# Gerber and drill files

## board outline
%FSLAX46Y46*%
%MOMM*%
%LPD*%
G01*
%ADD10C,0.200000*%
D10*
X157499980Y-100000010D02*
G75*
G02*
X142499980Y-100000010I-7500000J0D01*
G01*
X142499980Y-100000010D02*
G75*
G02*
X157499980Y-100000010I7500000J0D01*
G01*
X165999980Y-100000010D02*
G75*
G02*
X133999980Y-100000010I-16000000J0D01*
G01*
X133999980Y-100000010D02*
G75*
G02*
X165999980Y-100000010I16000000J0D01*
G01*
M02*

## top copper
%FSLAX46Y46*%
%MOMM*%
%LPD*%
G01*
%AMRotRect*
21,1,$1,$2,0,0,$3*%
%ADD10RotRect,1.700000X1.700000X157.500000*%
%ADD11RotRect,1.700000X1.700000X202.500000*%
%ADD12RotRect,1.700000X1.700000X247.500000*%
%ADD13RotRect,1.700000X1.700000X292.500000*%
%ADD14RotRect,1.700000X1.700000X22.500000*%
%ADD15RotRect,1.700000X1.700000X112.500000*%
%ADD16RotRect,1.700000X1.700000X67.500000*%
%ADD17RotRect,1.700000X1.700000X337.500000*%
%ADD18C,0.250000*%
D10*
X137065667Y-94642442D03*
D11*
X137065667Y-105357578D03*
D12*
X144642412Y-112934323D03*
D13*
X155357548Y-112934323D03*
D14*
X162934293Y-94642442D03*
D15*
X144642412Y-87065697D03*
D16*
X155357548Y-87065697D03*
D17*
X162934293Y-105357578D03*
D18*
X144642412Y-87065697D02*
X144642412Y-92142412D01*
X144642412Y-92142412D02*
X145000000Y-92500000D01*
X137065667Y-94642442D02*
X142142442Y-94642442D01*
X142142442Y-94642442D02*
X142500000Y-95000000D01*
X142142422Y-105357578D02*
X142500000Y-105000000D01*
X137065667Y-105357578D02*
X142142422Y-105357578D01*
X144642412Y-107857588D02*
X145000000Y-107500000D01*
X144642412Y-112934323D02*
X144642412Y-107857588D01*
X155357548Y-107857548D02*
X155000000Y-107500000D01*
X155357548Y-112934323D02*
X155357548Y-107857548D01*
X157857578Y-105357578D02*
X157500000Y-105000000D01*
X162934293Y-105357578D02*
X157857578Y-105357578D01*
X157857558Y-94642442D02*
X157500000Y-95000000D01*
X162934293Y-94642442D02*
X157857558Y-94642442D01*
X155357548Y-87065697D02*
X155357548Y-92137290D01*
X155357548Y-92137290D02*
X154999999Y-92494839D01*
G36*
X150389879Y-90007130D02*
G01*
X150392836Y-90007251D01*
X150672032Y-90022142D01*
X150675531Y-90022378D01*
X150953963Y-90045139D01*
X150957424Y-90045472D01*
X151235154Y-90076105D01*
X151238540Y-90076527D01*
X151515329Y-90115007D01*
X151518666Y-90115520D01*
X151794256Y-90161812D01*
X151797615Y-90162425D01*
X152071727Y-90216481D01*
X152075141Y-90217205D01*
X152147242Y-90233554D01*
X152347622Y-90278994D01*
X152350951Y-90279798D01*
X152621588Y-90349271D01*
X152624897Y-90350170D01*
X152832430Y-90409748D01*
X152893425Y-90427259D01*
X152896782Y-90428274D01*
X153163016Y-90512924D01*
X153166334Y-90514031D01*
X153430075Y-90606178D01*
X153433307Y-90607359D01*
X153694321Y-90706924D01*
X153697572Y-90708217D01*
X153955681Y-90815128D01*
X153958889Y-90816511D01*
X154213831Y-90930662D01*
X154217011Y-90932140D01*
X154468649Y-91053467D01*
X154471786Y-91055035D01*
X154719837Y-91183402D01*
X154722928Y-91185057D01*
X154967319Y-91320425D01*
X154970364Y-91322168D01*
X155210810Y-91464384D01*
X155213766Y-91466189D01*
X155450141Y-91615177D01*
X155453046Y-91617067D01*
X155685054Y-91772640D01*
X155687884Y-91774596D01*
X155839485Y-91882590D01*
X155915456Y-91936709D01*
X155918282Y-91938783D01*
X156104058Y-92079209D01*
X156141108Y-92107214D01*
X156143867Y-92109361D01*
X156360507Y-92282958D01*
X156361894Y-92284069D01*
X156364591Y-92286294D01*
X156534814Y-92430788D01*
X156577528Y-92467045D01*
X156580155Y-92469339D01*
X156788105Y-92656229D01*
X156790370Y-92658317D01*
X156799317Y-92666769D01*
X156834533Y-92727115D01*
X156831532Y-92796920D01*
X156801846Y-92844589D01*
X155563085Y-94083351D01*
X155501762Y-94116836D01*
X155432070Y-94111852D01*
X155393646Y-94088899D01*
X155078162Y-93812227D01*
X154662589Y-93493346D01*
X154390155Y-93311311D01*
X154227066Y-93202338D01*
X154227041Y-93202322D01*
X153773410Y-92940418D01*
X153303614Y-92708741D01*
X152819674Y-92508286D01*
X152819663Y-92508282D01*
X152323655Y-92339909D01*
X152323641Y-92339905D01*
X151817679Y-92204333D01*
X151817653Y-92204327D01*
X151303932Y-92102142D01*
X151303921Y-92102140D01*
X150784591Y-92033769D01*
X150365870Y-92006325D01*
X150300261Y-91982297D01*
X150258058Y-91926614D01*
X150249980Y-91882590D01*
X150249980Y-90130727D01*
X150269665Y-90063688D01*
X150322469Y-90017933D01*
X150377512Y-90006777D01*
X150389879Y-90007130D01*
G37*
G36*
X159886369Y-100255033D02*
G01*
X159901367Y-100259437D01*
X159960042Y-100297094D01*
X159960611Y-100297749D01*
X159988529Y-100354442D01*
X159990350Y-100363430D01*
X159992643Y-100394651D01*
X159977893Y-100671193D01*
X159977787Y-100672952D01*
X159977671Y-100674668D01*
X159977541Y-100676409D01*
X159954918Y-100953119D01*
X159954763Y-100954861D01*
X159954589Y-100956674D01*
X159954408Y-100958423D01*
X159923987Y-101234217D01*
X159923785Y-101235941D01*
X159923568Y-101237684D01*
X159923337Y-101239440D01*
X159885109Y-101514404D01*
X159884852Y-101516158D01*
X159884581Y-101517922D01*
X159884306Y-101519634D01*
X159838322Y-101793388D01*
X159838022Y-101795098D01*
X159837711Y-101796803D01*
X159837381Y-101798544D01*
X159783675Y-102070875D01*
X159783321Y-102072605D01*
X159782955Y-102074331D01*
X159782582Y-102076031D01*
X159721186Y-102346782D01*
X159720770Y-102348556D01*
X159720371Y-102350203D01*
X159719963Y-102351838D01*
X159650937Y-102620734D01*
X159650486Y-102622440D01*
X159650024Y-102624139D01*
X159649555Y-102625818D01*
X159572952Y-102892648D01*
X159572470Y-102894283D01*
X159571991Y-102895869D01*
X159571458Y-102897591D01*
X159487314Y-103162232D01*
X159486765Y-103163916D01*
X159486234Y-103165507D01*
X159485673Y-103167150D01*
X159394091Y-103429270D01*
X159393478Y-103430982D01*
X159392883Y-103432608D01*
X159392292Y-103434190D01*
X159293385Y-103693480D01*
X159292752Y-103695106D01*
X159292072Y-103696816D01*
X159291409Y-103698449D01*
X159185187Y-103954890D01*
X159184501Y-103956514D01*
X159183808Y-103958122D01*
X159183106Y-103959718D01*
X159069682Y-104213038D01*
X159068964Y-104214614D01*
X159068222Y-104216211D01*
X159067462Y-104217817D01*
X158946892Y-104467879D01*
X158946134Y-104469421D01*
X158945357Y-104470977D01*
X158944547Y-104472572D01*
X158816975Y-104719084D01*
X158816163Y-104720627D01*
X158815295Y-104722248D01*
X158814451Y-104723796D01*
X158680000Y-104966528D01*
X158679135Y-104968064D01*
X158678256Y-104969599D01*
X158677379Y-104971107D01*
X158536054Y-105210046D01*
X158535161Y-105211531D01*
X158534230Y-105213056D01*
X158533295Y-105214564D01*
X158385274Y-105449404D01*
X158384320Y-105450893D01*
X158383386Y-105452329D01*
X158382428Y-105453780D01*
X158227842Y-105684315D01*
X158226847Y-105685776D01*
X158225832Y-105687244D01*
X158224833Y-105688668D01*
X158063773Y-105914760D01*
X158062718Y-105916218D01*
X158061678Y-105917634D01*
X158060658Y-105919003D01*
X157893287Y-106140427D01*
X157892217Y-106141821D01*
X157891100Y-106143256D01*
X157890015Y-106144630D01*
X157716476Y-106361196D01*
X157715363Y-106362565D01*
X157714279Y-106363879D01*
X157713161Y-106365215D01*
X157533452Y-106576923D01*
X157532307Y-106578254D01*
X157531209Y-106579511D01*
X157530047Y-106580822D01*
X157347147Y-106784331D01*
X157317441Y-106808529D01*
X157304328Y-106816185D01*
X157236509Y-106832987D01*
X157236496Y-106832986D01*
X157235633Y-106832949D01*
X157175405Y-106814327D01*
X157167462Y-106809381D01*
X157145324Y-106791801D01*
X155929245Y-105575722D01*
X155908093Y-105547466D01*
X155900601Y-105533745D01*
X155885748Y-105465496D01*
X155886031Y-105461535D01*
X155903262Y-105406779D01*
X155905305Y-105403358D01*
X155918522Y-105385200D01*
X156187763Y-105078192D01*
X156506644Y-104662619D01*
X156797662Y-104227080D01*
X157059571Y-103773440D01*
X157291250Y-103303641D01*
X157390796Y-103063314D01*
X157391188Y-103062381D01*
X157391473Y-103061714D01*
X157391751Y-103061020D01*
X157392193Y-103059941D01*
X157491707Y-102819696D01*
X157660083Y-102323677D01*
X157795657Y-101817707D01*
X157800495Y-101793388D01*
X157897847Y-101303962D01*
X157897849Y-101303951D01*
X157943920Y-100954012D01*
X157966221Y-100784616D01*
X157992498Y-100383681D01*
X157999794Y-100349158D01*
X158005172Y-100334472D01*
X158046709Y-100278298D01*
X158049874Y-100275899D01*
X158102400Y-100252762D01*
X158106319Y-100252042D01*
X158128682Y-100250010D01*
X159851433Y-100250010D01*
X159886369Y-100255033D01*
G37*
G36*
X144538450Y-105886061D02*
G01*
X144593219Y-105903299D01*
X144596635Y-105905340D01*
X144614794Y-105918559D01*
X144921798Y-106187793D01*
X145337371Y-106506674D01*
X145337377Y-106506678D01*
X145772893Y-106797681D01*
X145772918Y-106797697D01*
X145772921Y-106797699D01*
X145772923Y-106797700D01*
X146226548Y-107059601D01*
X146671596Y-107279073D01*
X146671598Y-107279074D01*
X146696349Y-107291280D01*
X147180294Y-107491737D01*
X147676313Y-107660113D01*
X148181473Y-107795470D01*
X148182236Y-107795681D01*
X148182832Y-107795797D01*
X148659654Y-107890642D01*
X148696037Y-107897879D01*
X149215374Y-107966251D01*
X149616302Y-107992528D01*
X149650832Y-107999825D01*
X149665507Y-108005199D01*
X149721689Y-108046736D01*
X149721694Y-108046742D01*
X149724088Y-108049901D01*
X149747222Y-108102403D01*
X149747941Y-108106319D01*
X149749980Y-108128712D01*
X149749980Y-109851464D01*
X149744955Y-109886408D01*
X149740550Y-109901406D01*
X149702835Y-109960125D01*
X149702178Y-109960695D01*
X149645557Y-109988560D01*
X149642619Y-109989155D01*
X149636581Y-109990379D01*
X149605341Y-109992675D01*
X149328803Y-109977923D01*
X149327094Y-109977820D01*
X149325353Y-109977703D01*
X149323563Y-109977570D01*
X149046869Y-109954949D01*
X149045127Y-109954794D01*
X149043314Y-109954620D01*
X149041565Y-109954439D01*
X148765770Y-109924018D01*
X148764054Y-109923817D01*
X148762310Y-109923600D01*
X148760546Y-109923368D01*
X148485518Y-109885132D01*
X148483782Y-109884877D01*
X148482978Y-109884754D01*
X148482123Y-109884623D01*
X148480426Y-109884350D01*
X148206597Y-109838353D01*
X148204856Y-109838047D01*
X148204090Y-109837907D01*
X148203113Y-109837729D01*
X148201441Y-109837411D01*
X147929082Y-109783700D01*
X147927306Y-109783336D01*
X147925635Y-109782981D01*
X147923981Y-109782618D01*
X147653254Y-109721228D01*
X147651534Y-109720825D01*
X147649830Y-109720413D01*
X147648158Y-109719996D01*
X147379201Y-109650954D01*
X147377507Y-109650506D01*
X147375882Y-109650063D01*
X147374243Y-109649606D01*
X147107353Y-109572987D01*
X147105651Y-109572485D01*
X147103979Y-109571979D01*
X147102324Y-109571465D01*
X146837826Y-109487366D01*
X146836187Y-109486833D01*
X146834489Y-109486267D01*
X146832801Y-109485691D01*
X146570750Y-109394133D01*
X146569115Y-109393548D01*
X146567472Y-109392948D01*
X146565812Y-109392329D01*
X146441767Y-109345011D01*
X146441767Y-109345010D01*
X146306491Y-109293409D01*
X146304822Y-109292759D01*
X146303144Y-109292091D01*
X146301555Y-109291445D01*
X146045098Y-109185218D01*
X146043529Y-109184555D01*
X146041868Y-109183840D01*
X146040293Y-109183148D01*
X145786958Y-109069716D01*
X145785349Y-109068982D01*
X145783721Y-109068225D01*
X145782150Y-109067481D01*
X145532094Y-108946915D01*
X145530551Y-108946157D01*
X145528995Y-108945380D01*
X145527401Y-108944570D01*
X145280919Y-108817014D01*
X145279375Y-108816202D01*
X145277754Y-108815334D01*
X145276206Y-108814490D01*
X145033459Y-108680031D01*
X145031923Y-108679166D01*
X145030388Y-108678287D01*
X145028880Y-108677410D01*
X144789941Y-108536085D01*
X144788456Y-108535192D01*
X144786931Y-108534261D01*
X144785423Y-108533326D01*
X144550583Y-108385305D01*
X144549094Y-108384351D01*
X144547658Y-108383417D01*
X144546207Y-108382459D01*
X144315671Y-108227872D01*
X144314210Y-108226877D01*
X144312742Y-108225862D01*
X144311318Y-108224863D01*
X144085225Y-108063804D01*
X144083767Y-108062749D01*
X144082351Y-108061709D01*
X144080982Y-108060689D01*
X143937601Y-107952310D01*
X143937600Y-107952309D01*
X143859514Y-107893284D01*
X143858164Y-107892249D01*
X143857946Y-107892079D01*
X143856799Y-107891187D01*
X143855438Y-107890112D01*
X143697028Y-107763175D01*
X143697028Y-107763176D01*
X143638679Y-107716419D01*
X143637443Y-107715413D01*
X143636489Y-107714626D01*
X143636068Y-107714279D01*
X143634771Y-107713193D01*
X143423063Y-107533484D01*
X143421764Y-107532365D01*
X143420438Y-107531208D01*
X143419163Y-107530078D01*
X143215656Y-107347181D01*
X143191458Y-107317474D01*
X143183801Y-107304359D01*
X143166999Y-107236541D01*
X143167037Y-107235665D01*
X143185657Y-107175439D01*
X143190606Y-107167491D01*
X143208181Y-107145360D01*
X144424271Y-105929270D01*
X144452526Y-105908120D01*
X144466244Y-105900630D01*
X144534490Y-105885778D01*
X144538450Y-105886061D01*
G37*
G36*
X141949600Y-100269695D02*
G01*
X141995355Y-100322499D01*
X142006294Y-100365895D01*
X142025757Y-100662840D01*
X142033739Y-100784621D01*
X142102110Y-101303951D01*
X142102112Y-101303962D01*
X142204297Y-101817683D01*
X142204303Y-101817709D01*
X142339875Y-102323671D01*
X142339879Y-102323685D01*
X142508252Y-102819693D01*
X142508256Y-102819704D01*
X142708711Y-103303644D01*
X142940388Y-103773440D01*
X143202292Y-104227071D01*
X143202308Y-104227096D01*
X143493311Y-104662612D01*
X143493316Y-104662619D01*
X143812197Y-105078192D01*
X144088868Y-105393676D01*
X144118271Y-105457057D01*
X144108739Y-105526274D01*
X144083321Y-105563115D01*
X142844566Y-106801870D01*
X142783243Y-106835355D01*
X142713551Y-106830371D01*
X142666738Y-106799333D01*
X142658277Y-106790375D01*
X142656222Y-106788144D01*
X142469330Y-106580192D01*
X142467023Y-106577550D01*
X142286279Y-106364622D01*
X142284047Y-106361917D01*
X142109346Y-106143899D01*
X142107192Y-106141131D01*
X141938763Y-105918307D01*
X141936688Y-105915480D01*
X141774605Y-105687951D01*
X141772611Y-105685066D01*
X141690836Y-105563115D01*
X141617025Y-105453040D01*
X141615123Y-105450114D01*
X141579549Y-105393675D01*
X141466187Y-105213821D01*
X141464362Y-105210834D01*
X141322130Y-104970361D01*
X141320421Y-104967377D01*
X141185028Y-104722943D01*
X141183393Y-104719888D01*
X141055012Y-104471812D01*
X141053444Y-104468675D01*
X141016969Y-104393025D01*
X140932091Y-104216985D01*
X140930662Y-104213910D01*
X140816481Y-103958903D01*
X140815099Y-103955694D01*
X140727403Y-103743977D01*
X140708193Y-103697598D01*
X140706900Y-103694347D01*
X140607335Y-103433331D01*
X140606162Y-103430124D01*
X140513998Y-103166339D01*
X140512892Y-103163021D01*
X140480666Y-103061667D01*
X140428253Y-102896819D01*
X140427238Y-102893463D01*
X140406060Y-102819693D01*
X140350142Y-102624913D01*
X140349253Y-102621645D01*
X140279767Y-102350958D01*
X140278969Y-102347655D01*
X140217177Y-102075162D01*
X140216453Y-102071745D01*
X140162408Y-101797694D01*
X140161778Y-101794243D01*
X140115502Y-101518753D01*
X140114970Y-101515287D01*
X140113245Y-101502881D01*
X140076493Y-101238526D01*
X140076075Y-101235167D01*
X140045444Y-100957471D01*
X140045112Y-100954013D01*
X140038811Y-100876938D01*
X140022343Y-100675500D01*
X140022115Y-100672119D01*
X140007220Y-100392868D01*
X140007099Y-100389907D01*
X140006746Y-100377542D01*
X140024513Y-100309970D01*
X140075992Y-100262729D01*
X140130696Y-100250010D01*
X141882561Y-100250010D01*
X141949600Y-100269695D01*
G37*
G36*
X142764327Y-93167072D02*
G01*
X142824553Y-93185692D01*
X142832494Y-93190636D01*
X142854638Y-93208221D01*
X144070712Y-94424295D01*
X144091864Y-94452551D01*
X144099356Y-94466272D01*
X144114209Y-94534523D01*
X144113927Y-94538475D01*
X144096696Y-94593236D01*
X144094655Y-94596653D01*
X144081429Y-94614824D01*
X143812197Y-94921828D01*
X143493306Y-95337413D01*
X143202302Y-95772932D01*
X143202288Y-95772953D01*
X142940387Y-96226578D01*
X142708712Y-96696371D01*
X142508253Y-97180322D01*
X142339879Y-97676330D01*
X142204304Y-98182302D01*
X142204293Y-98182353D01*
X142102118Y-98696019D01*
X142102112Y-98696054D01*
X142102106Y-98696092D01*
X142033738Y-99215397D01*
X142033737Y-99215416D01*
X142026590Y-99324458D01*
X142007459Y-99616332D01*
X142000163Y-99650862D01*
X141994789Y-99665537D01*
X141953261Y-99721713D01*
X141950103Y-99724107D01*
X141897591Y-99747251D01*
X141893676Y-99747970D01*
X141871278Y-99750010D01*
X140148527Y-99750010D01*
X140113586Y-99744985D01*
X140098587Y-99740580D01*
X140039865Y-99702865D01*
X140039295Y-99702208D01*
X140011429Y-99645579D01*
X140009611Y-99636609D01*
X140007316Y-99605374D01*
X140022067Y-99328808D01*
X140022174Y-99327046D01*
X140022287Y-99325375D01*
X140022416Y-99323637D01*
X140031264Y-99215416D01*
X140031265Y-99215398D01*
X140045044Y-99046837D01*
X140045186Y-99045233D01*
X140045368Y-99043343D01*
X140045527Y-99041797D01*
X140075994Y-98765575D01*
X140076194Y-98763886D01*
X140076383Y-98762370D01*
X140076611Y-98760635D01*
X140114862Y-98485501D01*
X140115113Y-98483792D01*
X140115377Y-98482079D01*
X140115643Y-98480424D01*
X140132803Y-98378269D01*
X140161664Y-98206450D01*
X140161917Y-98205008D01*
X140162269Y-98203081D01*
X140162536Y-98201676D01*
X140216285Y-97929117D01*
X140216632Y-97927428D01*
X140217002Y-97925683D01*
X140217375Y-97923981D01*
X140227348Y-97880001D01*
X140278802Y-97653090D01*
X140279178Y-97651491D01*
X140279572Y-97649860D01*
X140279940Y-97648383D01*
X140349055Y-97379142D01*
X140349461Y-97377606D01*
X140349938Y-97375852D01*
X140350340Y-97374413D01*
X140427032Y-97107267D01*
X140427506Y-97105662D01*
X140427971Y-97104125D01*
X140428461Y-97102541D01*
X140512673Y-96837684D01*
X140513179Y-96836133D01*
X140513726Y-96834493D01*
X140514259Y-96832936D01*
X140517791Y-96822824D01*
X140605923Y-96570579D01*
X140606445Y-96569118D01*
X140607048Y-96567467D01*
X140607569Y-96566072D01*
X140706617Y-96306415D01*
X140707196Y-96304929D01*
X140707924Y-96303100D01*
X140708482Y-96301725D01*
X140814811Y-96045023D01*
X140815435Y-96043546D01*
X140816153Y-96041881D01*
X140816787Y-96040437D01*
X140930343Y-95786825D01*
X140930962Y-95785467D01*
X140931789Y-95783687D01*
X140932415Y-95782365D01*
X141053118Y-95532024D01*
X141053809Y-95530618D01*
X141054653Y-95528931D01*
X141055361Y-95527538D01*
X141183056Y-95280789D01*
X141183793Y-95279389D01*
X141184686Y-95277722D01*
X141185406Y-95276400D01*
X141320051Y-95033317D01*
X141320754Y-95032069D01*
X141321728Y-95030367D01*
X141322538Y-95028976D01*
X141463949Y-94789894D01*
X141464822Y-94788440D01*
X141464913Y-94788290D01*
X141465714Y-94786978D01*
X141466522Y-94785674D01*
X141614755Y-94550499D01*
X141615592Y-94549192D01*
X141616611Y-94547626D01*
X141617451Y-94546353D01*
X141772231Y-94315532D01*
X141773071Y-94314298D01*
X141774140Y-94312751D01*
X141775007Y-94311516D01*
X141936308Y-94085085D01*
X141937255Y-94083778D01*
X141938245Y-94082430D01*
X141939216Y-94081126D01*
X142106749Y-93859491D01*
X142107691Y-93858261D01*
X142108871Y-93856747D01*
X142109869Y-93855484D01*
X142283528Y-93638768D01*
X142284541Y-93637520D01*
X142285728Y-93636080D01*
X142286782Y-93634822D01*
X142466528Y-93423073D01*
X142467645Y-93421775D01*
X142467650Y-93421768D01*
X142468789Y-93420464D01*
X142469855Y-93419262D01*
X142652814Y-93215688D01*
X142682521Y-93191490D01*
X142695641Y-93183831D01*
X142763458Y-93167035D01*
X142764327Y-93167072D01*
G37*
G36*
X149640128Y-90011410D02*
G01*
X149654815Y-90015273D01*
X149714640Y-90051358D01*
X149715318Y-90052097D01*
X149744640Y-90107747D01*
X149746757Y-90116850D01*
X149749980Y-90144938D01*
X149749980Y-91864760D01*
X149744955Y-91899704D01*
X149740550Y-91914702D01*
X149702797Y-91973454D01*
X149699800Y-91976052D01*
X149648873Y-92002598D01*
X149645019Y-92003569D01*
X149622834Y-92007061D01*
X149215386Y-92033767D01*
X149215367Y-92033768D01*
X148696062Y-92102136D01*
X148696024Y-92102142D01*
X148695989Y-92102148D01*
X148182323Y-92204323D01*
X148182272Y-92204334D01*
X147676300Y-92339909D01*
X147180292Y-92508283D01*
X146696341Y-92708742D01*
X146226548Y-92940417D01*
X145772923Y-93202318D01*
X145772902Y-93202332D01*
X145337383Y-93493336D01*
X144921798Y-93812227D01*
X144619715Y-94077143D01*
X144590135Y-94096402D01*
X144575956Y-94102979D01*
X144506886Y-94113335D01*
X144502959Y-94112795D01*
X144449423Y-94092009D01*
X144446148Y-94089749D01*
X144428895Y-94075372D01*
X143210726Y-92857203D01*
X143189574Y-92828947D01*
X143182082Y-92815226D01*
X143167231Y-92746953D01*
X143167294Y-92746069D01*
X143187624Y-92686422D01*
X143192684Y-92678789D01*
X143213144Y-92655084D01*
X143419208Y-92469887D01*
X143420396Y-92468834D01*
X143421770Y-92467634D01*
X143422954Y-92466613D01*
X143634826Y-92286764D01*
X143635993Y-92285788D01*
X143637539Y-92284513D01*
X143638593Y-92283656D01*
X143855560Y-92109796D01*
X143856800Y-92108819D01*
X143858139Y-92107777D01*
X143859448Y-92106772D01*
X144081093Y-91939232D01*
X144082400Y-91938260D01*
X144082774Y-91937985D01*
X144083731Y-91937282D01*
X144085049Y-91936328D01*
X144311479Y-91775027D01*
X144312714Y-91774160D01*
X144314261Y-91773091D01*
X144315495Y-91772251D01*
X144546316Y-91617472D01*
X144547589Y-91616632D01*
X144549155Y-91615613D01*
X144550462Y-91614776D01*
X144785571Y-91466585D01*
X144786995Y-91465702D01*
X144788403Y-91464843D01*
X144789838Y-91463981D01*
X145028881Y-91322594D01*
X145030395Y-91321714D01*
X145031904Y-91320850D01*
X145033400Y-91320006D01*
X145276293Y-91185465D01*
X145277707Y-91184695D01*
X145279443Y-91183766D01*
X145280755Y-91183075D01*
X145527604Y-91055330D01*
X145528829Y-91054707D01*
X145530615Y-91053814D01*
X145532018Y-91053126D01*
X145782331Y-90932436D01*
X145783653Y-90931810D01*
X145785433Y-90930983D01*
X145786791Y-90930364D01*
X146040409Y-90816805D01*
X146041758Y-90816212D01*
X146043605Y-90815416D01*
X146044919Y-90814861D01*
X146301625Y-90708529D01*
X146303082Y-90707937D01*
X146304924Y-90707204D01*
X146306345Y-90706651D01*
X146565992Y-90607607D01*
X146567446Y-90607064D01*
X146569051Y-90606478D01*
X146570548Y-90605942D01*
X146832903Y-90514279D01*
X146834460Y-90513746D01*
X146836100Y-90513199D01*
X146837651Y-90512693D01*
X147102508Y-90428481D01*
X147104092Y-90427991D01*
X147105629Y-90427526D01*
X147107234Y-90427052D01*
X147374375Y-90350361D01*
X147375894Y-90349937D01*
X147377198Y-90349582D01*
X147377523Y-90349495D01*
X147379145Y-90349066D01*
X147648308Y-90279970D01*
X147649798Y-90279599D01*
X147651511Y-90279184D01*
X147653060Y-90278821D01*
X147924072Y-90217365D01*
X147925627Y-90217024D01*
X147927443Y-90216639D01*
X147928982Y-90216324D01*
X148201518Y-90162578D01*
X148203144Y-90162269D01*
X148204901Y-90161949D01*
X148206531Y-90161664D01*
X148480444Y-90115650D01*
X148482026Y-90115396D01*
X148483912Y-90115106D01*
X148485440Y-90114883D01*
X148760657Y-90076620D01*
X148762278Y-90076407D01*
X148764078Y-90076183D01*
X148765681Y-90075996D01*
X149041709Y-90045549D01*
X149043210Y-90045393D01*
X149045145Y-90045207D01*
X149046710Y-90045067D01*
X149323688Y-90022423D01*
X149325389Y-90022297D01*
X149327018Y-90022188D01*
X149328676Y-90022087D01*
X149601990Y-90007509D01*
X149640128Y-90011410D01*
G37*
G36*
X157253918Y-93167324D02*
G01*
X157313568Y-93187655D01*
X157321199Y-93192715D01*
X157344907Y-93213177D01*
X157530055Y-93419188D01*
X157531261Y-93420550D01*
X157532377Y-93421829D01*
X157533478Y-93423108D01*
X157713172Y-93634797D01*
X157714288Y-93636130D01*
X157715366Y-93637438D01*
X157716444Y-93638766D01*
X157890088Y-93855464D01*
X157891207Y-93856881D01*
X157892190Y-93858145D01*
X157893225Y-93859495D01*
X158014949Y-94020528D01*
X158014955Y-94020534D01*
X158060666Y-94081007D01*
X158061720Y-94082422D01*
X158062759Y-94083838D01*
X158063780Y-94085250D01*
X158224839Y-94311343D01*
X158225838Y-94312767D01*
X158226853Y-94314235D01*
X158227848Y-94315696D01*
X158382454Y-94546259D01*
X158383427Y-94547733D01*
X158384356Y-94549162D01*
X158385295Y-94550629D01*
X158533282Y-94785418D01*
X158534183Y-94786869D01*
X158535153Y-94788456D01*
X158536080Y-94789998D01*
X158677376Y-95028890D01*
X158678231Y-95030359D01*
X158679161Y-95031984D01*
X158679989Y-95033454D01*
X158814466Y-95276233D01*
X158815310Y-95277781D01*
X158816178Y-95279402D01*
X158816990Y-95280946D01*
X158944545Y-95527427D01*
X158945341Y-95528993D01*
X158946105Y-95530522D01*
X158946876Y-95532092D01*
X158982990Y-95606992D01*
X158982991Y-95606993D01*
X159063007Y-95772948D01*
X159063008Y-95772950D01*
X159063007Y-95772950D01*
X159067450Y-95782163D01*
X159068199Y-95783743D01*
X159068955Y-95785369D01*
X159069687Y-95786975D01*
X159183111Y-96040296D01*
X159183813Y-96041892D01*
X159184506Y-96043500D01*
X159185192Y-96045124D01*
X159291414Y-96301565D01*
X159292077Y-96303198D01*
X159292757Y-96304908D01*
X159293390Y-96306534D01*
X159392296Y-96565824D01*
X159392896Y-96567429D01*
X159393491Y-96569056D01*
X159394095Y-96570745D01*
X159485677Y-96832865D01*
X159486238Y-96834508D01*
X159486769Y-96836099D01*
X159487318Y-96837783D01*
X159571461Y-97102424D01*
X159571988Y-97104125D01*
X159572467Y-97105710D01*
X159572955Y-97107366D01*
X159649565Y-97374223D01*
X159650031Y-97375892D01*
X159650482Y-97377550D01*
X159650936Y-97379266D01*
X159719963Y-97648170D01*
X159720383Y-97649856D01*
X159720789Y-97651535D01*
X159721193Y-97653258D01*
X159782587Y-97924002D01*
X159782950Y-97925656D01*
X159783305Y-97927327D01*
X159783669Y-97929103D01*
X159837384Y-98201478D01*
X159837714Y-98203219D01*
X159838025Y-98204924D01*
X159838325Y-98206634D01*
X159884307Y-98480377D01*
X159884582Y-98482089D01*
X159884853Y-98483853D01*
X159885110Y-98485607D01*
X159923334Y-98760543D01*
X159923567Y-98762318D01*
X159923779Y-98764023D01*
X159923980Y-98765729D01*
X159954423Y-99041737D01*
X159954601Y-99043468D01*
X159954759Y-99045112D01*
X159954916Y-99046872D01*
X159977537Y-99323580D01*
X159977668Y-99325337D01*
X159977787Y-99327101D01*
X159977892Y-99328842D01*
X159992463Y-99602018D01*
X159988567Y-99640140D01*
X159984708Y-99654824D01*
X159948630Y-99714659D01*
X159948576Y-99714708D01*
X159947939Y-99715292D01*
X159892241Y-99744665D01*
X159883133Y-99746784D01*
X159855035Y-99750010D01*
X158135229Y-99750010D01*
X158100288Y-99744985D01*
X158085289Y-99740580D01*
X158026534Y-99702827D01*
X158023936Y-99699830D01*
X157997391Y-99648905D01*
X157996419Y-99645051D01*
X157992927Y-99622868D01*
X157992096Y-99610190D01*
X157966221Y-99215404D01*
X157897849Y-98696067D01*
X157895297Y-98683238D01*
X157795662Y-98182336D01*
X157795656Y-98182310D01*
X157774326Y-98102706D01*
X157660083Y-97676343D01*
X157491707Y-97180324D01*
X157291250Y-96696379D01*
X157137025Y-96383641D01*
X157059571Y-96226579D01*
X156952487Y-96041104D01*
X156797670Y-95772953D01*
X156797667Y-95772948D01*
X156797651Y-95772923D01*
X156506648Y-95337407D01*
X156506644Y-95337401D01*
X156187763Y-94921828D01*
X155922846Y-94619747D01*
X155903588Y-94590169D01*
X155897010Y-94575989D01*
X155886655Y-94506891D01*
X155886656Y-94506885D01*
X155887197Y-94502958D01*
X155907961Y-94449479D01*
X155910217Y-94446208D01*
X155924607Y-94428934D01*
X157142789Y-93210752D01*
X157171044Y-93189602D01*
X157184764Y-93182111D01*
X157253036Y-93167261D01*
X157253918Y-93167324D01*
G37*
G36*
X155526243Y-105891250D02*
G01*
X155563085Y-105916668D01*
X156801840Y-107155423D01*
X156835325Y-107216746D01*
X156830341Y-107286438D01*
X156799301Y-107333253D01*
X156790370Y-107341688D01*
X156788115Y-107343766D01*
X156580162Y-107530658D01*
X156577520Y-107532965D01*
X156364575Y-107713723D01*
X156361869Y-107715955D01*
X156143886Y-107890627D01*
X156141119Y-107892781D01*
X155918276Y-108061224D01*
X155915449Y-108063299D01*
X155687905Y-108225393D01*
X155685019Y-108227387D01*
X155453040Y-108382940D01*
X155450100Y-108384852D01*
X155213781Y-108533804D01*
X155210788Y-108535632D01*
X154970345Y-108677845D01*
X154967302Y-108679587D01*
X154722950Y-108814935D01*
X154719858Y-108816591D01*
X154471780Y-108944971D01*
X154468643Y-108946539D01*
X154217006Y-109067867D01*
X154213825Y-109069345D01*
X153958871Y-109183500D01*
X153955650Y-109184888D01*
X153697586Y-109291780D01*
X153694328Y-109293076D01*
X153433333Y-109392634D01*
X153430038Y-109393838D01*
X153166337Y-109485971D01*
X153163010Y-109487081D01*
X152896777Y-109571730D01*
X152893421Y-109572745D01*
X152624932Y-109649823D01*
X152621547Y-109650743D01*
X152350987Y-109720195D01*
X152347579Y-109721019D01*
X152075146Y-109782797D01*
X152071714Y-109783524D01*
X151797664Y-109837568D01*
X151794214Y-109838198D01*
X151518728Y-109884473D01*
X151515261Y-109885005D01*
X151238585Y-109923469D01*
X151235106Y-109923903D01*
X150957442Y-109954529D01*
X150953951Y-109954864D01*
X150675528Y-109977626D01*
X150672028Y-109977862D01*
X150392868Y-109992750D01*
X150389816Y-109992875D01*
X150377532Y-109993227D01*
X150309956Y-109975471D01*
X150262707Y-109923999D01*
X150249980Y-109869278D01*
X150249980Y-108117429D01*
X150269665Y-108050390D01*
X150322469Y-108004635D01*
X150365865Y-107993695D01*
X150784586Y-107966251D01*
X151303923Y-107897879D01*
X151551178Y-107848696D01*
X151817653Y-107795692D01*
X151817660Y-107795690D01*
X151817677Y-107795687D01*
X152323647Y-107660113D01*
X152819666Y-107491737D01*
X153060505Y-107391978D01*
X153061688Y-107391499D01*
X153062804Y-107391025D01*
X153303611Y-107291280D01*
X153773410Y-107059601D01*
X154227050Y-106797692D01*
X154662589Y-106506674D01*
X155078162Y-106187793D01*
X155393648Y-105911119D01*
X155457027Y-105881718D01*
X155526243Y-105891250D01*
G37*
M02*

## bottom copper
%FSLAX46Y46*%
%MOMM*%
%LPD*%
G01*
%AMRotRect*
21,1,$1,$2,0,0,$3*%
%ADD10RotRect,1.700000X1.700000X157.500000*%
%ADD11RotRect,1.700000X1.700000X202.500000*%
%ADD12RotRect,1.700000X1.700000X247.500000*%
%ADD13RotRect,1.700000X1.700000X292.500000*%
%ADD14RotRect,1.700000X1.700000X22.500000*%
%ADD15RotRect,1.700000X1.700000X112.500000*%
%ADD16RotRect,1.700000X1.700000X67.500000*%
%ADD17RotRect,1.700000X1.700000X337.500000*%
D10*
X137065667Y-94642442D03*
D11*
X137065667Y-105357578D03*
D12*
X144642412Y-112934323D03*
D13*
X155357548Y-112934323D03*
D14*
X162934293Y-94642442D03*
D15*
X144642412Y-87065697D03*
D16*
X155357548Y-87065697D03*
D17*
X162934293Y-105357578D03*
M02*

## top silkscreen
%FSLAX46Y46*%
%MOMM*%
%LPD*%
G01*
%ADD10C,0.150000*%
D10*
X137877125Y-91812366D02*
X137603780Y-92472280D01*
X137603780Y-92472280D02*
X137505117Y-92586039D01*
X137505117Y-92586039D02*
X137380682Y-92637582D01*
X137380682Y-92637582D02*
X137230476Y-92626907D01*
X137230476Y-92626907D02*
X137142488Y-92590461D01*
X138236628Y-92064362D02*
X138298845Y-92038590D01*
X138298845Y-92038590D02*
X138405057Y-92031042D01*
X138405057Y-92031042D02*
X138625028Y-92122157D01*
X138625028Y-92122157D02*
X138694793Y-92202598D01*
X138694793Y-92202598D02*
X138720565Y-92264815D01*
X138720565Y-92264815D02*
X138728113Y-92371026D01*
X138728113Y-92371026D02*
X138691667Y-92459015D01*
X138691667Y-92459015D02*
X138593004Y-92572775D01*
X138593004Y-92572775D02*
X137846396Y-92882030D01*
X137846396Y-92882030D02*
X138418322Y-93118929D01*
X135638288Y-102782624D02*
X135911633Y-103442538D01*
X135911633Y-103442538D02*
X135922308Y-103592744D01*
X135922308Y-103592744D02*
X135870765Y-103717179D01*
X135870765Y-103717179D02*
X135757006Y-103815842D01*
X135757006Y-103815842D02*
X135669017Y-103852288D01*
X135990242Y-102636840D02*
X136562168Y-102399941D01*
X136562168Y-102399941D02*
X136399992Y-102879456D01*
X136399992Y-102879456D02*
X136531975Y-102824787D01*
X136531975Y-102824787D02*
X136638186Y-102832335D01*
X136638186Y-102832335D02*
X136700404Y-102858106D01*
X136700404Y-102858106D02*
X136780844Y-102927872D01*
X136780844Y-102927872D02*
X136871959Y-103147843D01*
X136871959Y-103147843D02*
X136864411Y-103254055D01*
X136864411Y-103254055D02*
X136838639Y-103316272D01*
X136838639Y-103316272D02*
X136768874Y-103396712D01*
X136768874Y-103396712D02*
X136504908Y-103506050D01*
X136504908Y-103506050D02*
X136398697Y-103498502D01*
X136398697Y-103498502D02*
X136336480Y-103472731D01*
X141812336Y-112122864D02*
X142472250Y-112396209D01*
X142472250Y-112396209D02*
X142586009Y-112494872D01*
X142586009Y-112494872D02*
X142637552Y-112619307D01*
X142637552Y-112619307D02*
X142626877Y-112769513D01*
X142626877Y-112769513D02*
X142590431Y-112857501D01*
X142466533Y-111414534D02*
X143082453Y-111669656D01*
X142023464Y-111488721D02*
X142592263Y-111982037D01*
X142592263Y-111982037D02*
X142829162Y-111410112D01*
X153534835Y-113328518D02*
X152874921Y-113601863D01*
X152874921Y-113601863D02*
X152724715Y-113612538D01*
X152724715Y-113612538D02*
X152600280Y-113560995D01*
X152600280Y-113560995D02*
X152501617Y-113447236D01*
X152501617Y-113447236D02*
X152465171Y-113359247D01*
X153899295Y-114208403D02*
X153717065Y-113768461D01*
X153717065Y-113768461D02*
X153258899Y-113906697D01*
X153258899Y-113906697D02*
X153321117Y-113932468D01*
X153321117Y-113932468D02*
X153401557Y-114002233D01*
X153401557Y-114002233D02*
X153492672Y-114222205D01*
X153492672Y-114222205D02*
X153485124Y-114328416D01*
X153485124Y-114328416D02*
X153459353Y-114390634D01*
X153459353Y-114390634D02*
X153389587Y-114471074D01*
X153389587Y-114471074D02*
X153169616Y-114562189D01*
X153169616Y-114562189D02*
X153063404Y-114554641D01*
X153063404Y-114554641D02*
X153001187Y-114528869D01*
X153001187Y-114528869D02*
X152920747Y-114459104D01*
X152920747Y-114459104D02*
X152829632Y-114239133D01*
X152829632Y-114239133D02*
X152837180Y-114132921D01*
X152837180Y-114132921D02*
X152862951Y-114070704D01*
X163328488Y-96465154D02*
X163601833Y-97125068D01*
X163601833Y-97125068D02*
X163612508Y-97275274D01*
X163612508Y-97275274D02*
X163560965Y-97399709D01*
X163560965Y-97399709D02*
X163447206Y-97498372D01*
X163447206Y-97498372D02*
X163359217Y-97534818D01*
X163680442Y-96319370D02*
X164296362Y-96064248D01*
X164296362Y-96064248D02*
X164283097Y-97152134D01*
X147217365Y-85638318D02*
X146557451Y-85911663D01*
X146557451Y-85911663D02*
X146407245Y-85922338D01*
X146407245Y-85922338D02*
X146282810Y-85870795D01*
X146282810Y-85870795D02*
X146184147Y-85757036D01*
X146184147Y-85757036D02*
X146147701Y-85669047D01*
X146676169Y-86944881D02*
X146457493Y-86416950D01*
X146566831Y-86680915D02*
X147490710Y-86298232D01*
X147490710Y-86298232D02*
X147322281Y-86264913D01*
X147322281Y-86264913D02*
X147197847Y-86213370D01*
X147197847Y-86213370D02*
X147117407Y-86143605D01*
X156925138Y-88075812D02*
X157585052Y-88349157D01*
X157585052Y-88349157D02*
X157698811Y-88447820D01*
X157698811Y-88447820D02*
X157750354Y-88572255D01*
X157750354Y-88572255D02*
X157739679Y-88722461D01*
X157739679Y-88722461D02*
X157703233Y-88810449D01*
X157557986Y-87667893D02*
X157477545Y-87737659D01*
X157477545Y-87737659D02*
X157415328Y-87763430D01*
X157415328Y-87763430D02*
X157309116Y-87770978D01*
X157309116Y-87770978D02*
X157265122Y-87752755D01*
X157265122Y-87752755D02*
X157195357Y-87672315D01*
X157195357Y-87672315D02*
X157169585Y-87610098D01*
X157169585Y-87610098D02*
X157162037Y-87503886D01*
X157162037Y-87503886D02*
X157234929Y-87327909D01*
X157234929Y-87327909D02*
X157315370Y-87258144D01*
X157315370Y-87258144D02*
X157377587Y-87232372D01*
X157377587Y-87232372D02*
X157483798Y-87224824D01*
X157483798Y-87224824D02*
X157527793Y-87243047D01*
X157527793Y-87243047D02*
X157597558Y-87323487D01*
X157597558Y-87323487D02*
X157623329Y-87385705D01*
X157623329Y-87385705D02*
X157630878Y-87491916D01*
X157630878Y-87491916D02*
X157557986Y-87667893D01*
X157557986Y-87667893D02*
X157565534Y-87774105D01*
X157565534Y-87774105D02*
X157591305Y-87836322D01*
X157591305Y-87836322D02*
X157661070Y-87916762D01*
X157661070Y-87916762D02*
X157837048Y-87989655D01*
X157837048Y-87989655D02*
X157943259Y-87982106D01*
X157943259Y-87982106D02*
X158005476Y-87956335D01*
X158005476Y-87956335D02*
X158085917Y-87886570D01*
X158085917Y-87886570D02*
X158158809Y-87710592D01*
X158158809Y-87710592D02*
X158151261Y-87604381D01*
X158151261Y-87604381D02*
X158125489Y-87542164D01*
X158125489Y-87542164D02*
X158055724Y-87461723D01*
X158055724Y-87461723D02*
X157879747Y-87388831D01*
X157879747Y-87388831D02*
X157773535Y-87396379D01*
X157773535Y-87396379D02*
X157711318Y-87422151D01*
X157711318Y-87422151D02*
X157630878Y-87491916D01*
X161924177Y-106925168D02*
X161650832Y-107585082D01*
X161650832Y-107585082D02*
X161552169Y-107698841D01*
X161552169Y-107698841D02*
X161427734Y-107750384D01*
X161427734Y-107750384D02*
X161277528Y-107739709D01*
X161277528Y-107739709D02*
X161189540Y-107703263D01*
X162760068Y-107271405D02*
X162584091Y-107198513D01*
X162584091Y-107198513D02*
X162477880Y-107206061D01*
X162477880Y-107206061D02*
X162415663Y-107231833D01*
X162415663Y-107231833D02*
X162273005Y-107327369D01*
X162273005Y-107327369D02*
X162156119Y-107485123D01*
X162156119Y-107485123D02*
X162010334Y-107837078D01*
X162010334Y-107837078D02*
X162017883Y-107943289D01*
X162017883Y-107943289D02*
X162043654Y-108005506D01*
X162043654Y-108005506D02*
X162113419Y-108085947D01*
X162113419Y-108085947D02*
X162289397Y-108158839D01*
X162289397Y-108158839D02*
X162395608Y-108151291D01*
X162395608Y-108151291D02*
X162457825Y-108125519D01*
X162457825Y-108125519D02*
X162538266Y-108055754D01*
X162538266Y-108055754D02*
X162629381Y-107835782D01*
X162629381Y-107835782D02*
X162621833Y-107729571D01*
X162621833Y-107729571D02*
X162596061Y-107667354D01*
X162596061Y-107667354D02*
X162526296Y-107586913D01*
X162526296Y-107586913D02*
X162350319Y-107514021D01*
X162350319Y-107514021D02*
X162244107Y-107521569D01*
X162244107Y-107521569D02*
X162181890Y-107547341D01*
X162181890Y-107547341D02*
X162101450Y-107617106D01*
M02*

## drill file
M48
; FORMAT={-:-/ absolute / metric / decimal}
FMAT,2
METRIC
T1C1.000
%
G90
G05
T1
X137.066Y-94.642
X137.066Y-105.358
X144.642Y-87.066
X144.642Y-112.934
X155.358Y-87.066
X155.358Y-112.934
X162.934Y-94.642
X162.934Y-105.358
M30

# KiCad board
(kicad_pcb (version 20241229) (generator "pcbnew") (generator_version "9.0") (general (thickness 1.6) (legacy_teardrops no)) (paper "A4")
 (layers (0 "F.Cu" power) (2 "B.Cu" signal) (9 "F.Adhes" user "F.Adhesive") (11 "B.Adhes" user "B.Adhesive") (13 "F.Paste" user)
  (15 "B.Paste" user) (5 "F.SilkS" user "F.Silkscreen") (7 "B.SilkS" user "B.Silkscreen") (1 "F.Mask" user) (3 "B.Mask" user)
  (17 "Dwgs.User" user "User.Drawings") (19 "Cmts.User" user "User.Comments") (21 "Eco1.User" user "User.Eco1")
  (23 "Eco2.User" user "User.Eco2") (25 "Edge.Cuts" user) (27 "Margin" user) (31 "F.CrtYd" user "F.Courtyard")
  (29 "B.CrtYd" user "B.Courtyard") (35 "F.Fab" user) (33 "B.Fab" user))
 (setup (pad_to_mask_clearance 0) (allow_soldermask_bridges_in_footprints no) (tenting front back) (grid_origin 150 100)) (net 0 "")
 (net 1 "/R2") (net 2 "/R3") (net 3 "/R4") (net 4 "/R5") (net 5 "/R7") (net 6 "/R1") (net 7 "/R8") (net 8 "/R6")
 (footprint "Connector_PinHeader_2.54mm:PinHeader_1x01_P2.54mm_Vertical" (layer "B.Cu") (at 137.065667 94.642442 157.5)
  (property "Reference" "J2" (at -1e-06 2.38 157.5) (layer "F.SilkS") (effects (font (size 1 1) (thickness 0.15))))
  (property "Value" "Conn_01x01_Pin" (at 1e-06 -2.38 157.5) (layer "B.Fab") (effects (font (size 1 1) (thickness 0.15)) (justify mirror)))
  (pad "1" thru_hole rect (at 0 0 157.5) (size 1.7 1.7) (drill 1) (layers "*.Cu" "*.Mask") (remove_unused_layers no) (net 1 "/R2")))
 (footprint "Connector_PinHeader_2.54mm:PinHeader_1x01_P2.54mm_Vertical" (layer "B.Cu") (at 137.065667 105.357578 -157.5)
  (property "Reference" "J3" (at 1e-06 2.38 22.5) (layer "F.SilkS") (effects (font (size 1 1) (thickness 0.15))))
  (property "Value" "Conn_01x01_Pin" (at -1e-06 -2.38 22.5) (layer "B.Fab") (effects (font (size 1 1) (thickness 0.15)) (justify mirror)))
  (pad "1" thru_hole rect (at 0 0 202.5) (size 1.7 1.7) (drill 1) (layers "*.Cu" "*.Mask") (remove_unused_layers no) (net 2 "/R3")))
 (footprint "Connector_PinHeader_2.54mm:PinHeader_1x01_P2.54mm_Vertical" (layer "B.Cu") (at 144.642412 112.934323 -112.5)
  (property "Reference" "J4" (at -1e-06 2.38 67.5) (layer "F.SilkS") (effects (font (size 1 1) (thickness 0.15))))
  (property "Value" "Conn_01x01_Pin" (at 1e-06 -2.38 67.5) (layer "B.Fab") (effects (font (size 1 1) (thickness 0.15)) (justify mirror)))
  (pad "1" thru_hole rect (at 0 0 247.5) (size 1.7 1.7) (drill 1) (layers "*.Cu" "*.Mask") (remove_unused_layers no) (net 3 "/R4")))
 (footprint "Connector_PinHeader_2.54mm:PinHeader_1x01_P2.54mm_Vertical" (layer "B.Cu") (at 155.357548 112.934323 -67.5)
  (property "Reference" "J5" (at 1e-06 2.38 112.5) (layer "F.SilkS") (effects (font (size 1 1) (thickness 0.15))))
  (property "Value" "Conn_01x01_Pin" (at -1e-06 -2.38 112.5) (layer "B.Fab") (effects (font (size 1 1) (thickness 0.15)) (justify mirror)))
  (pad "1" thru_hole rect (at 0 0 292.5) (size 1.7 1.7) (drill 1) (layers "*.Cu" "*.Mask") (remove_unused_layers no) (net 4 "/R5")))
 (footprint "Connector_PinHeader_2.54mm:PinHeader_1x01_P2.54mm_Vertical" (layer "B.Cu") (at 162.934293 94.642442 22.5)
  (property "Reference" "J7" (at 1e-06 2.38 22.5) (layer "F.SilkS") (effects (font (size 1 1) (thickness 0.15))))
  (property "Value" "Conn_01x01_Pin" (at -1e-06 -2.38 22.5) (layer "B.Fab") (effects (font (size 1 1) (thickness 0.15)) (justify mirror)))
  (pad "1" thru_hole rect (at 0 0 22.5) (size 1.7 1.7) (drill 1) (layers "*.Cu" "*.Mask") (remove_unused_layers no) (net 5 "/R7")))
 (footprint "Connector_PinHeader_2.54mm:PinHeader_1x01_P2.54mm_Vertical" (layer "B.Cu") (at 144.642412 87.065697 112.5)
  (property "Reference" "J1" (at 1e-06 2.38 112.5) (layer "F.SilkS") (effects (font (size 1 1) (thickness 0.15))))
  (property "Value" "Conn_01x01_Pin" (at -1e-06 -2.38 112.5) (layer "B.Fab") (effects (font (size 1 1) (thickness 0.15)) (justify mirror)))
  (pad "1" thru_hole rect (at 0 0 112.5) (size 1.7 1.7) (drill 1) (layers "*.Cu" "*.Mask") (remove_unused_layers no) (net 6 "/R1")))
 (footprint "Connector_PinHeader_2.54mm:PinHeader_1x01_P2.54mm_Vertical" (layer "B.Cu") (at 155.357548 87.065697 67.5)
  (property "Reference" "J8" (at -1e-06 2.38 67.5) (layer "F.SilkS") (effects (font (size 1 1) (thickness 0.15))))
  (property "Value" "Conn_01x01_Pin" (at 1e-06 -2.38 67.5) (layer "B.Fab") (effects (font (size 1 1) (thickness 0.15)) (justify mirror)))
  (pad "1" thru_hole rect (at 0 0 67.5) (size 1.7 1.7) (drill 1) (layers "*.Cu" "*.Mask") (remove_unused_layers no) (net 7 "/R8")))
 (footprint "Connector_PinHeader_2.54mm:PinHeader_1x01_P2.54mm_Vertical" (layer "B.Cu") (at 162.934293 105.357578 -22.5)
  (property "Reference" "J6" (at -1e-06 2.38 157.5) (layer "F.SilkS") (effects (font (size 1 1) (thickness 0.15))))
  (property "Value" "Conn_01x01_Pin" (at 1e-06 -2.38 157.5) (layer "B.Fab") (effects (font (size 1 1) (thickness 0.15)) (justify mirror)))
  (pad "1" thru_hole rect (at 0 0 337.5) (size 1.7 1.7) (drill 1) (layers "*.Cu" "*.Mask") (remove_unused_layers no) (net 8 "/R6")))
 (gr_circle (center 149.99998 100.00001) (end 157.49998 100.00001) (stroke (width 0.2) (type solid)) (fill no) (layer "Edge.Cuts"))
 (gr_circle (center 149.99998 100.00001) (end 165.99998 100.00001) (stroke (width 0.2) (type solid)) (fill no) (layer "Edge.Cuts"))
 (segment (start 144.642412 87.065697) (end 144.642412 92.14241199999999) (width 0.25) (layer "F.Cu") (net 6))
 (segment (start 144.642412 92.14241199999999) (end 145 92.5) (width 0.25) (layer "F.Cu") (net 6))
 (segment (start 137.065667 94.642442) (end 142.142442 94.642442) (width 0.25) (layer "F.Cu") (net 1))
 (segment (start 142.142442 94.642442) (end 142.5 95) (width 0.25) (layer "F.Cu") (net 1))
 (segment (start 142.142422 105.357578) (end 142.5 105) (width 0.25) (layer "F.Cu") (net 2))
 (segment (start 137.065667 105.357578) (end 142.142422 105.357578) (width 0.25) (layer "F.Cu") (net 2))
 (segment (start 144.642412 107.857588) (end 145 107.5) (width 0.25) (layer "F.Cu") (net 3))
 (segment (start 144.642412 112.934323) (end 144.642412 107.857588) (width 0.25) (layer "F.Cu") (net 3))
 (segment (start 155.357548 107.857548) (end 155 107.5) (width 0.25) (layer "F.Cu") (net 4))
 (segment (start 155.357548 112.934323) (end 155.357548 107.857548) (width 0.25) (layer "F.Cu") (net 4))
 (segment (start 157.857578 105.357578) (end 157.5 105) (width 0.25) (layer "F.Cu") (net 8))
 (segment (start 162.934293 105.357578) (end 157.857578 105.357578) (width 0.25) (layer "F.Cu") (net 8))
 (segment (start 157.857558 94.642442) (end 157.5 95) (width 0.25) (layer "F.Cu") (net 5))
 (segment (start 162.934293 94.642442) (end 157.857558 94.642442) (width 0.25) (layer "F.Cu") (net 5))
 (segment (start 155.357548 87.065697) (end 155.357548 92.13728999999999) (width 0.25) (layer "F.Cu") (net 7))
 (segment (start 155.357548 92.13728999999999) (end 154.999999 92.494839) (width 0.25) (layer "F.Cu") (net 7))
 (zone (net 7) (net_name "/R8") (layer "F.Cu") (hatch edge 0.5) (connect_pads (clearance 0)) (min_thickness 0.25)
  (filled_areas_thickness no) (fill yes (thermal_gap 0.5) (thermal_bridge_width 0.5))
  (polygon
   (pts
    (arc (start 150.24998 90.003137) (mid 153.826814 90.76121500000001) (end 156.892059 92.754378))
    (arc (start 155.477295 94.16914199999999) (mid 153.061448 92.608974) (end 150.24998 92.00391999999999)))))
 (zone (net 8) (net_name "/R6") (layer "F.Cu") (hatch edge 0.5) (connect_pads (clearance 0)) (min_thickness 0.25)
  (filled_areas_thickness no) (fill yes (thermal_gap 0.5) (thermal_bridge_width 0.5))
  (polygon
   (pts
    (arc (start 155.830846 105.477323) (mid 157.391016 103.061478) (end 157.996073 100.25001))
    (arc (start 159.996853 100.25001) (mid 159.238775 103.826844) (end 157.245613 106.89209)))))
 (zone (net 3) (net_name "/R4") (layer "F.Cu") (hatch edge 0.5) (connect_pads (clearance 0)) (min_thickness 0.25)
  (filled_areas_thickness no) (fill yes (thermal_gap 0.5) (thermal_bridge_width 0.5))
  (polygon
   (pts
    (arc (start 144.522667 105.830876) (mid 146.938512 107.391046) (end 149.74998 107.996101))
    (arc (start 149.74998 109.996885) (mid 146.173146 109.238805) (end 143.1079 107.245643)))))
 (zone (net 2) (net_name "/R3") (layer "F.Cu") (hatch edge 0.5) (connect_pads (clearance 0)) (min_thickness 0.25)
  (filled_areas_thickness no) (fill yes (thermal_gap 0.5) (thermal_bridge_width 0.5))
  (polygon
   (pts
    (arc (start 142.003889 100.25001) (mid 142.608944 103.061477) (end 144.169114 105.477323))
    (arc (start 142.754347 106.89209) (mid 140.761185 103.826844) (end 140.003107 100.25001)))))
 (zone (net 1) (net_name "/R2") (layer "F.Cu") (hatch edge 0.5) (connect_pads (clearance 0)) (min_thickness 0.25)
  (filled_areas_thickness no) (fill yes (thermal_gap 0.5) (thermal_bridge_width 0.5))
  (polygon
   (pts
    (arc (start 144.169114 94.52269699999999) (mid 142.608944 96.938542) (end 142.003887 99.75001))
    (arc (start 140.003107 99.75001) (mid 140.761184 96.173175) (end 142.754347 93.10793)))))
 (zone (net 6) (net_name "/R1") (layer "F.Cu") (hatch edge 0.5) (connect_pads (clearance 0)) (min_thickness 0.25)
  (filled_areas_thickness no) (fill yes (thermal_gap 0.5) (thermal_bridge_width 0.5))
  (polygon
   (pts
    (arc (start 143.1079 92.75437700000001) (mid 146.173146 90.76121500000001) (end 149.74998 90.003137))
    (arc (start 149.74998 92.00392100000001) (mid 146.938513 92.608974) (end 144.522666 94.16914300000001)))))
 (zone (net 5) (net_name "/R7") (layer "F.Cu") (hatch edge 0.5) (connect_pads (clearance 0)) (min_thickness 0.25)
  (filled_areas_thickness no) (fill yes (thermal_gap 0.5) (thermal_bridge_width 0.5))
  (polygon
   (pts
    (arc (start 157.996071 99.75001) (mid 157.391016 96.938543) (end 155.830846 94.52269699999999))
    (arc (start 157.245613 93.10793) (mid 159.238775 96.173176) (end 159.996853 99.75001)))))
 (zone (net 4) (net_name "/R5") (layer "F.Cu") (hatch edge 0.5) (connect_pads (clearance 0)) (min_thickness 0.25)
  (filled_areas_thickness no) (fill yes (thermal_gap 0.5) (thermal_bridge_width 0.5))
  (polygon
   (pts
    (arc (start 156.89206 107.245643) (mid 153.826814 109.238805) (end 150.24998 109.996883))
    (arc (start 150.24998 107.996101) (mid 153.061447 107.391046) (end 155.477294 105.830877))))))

